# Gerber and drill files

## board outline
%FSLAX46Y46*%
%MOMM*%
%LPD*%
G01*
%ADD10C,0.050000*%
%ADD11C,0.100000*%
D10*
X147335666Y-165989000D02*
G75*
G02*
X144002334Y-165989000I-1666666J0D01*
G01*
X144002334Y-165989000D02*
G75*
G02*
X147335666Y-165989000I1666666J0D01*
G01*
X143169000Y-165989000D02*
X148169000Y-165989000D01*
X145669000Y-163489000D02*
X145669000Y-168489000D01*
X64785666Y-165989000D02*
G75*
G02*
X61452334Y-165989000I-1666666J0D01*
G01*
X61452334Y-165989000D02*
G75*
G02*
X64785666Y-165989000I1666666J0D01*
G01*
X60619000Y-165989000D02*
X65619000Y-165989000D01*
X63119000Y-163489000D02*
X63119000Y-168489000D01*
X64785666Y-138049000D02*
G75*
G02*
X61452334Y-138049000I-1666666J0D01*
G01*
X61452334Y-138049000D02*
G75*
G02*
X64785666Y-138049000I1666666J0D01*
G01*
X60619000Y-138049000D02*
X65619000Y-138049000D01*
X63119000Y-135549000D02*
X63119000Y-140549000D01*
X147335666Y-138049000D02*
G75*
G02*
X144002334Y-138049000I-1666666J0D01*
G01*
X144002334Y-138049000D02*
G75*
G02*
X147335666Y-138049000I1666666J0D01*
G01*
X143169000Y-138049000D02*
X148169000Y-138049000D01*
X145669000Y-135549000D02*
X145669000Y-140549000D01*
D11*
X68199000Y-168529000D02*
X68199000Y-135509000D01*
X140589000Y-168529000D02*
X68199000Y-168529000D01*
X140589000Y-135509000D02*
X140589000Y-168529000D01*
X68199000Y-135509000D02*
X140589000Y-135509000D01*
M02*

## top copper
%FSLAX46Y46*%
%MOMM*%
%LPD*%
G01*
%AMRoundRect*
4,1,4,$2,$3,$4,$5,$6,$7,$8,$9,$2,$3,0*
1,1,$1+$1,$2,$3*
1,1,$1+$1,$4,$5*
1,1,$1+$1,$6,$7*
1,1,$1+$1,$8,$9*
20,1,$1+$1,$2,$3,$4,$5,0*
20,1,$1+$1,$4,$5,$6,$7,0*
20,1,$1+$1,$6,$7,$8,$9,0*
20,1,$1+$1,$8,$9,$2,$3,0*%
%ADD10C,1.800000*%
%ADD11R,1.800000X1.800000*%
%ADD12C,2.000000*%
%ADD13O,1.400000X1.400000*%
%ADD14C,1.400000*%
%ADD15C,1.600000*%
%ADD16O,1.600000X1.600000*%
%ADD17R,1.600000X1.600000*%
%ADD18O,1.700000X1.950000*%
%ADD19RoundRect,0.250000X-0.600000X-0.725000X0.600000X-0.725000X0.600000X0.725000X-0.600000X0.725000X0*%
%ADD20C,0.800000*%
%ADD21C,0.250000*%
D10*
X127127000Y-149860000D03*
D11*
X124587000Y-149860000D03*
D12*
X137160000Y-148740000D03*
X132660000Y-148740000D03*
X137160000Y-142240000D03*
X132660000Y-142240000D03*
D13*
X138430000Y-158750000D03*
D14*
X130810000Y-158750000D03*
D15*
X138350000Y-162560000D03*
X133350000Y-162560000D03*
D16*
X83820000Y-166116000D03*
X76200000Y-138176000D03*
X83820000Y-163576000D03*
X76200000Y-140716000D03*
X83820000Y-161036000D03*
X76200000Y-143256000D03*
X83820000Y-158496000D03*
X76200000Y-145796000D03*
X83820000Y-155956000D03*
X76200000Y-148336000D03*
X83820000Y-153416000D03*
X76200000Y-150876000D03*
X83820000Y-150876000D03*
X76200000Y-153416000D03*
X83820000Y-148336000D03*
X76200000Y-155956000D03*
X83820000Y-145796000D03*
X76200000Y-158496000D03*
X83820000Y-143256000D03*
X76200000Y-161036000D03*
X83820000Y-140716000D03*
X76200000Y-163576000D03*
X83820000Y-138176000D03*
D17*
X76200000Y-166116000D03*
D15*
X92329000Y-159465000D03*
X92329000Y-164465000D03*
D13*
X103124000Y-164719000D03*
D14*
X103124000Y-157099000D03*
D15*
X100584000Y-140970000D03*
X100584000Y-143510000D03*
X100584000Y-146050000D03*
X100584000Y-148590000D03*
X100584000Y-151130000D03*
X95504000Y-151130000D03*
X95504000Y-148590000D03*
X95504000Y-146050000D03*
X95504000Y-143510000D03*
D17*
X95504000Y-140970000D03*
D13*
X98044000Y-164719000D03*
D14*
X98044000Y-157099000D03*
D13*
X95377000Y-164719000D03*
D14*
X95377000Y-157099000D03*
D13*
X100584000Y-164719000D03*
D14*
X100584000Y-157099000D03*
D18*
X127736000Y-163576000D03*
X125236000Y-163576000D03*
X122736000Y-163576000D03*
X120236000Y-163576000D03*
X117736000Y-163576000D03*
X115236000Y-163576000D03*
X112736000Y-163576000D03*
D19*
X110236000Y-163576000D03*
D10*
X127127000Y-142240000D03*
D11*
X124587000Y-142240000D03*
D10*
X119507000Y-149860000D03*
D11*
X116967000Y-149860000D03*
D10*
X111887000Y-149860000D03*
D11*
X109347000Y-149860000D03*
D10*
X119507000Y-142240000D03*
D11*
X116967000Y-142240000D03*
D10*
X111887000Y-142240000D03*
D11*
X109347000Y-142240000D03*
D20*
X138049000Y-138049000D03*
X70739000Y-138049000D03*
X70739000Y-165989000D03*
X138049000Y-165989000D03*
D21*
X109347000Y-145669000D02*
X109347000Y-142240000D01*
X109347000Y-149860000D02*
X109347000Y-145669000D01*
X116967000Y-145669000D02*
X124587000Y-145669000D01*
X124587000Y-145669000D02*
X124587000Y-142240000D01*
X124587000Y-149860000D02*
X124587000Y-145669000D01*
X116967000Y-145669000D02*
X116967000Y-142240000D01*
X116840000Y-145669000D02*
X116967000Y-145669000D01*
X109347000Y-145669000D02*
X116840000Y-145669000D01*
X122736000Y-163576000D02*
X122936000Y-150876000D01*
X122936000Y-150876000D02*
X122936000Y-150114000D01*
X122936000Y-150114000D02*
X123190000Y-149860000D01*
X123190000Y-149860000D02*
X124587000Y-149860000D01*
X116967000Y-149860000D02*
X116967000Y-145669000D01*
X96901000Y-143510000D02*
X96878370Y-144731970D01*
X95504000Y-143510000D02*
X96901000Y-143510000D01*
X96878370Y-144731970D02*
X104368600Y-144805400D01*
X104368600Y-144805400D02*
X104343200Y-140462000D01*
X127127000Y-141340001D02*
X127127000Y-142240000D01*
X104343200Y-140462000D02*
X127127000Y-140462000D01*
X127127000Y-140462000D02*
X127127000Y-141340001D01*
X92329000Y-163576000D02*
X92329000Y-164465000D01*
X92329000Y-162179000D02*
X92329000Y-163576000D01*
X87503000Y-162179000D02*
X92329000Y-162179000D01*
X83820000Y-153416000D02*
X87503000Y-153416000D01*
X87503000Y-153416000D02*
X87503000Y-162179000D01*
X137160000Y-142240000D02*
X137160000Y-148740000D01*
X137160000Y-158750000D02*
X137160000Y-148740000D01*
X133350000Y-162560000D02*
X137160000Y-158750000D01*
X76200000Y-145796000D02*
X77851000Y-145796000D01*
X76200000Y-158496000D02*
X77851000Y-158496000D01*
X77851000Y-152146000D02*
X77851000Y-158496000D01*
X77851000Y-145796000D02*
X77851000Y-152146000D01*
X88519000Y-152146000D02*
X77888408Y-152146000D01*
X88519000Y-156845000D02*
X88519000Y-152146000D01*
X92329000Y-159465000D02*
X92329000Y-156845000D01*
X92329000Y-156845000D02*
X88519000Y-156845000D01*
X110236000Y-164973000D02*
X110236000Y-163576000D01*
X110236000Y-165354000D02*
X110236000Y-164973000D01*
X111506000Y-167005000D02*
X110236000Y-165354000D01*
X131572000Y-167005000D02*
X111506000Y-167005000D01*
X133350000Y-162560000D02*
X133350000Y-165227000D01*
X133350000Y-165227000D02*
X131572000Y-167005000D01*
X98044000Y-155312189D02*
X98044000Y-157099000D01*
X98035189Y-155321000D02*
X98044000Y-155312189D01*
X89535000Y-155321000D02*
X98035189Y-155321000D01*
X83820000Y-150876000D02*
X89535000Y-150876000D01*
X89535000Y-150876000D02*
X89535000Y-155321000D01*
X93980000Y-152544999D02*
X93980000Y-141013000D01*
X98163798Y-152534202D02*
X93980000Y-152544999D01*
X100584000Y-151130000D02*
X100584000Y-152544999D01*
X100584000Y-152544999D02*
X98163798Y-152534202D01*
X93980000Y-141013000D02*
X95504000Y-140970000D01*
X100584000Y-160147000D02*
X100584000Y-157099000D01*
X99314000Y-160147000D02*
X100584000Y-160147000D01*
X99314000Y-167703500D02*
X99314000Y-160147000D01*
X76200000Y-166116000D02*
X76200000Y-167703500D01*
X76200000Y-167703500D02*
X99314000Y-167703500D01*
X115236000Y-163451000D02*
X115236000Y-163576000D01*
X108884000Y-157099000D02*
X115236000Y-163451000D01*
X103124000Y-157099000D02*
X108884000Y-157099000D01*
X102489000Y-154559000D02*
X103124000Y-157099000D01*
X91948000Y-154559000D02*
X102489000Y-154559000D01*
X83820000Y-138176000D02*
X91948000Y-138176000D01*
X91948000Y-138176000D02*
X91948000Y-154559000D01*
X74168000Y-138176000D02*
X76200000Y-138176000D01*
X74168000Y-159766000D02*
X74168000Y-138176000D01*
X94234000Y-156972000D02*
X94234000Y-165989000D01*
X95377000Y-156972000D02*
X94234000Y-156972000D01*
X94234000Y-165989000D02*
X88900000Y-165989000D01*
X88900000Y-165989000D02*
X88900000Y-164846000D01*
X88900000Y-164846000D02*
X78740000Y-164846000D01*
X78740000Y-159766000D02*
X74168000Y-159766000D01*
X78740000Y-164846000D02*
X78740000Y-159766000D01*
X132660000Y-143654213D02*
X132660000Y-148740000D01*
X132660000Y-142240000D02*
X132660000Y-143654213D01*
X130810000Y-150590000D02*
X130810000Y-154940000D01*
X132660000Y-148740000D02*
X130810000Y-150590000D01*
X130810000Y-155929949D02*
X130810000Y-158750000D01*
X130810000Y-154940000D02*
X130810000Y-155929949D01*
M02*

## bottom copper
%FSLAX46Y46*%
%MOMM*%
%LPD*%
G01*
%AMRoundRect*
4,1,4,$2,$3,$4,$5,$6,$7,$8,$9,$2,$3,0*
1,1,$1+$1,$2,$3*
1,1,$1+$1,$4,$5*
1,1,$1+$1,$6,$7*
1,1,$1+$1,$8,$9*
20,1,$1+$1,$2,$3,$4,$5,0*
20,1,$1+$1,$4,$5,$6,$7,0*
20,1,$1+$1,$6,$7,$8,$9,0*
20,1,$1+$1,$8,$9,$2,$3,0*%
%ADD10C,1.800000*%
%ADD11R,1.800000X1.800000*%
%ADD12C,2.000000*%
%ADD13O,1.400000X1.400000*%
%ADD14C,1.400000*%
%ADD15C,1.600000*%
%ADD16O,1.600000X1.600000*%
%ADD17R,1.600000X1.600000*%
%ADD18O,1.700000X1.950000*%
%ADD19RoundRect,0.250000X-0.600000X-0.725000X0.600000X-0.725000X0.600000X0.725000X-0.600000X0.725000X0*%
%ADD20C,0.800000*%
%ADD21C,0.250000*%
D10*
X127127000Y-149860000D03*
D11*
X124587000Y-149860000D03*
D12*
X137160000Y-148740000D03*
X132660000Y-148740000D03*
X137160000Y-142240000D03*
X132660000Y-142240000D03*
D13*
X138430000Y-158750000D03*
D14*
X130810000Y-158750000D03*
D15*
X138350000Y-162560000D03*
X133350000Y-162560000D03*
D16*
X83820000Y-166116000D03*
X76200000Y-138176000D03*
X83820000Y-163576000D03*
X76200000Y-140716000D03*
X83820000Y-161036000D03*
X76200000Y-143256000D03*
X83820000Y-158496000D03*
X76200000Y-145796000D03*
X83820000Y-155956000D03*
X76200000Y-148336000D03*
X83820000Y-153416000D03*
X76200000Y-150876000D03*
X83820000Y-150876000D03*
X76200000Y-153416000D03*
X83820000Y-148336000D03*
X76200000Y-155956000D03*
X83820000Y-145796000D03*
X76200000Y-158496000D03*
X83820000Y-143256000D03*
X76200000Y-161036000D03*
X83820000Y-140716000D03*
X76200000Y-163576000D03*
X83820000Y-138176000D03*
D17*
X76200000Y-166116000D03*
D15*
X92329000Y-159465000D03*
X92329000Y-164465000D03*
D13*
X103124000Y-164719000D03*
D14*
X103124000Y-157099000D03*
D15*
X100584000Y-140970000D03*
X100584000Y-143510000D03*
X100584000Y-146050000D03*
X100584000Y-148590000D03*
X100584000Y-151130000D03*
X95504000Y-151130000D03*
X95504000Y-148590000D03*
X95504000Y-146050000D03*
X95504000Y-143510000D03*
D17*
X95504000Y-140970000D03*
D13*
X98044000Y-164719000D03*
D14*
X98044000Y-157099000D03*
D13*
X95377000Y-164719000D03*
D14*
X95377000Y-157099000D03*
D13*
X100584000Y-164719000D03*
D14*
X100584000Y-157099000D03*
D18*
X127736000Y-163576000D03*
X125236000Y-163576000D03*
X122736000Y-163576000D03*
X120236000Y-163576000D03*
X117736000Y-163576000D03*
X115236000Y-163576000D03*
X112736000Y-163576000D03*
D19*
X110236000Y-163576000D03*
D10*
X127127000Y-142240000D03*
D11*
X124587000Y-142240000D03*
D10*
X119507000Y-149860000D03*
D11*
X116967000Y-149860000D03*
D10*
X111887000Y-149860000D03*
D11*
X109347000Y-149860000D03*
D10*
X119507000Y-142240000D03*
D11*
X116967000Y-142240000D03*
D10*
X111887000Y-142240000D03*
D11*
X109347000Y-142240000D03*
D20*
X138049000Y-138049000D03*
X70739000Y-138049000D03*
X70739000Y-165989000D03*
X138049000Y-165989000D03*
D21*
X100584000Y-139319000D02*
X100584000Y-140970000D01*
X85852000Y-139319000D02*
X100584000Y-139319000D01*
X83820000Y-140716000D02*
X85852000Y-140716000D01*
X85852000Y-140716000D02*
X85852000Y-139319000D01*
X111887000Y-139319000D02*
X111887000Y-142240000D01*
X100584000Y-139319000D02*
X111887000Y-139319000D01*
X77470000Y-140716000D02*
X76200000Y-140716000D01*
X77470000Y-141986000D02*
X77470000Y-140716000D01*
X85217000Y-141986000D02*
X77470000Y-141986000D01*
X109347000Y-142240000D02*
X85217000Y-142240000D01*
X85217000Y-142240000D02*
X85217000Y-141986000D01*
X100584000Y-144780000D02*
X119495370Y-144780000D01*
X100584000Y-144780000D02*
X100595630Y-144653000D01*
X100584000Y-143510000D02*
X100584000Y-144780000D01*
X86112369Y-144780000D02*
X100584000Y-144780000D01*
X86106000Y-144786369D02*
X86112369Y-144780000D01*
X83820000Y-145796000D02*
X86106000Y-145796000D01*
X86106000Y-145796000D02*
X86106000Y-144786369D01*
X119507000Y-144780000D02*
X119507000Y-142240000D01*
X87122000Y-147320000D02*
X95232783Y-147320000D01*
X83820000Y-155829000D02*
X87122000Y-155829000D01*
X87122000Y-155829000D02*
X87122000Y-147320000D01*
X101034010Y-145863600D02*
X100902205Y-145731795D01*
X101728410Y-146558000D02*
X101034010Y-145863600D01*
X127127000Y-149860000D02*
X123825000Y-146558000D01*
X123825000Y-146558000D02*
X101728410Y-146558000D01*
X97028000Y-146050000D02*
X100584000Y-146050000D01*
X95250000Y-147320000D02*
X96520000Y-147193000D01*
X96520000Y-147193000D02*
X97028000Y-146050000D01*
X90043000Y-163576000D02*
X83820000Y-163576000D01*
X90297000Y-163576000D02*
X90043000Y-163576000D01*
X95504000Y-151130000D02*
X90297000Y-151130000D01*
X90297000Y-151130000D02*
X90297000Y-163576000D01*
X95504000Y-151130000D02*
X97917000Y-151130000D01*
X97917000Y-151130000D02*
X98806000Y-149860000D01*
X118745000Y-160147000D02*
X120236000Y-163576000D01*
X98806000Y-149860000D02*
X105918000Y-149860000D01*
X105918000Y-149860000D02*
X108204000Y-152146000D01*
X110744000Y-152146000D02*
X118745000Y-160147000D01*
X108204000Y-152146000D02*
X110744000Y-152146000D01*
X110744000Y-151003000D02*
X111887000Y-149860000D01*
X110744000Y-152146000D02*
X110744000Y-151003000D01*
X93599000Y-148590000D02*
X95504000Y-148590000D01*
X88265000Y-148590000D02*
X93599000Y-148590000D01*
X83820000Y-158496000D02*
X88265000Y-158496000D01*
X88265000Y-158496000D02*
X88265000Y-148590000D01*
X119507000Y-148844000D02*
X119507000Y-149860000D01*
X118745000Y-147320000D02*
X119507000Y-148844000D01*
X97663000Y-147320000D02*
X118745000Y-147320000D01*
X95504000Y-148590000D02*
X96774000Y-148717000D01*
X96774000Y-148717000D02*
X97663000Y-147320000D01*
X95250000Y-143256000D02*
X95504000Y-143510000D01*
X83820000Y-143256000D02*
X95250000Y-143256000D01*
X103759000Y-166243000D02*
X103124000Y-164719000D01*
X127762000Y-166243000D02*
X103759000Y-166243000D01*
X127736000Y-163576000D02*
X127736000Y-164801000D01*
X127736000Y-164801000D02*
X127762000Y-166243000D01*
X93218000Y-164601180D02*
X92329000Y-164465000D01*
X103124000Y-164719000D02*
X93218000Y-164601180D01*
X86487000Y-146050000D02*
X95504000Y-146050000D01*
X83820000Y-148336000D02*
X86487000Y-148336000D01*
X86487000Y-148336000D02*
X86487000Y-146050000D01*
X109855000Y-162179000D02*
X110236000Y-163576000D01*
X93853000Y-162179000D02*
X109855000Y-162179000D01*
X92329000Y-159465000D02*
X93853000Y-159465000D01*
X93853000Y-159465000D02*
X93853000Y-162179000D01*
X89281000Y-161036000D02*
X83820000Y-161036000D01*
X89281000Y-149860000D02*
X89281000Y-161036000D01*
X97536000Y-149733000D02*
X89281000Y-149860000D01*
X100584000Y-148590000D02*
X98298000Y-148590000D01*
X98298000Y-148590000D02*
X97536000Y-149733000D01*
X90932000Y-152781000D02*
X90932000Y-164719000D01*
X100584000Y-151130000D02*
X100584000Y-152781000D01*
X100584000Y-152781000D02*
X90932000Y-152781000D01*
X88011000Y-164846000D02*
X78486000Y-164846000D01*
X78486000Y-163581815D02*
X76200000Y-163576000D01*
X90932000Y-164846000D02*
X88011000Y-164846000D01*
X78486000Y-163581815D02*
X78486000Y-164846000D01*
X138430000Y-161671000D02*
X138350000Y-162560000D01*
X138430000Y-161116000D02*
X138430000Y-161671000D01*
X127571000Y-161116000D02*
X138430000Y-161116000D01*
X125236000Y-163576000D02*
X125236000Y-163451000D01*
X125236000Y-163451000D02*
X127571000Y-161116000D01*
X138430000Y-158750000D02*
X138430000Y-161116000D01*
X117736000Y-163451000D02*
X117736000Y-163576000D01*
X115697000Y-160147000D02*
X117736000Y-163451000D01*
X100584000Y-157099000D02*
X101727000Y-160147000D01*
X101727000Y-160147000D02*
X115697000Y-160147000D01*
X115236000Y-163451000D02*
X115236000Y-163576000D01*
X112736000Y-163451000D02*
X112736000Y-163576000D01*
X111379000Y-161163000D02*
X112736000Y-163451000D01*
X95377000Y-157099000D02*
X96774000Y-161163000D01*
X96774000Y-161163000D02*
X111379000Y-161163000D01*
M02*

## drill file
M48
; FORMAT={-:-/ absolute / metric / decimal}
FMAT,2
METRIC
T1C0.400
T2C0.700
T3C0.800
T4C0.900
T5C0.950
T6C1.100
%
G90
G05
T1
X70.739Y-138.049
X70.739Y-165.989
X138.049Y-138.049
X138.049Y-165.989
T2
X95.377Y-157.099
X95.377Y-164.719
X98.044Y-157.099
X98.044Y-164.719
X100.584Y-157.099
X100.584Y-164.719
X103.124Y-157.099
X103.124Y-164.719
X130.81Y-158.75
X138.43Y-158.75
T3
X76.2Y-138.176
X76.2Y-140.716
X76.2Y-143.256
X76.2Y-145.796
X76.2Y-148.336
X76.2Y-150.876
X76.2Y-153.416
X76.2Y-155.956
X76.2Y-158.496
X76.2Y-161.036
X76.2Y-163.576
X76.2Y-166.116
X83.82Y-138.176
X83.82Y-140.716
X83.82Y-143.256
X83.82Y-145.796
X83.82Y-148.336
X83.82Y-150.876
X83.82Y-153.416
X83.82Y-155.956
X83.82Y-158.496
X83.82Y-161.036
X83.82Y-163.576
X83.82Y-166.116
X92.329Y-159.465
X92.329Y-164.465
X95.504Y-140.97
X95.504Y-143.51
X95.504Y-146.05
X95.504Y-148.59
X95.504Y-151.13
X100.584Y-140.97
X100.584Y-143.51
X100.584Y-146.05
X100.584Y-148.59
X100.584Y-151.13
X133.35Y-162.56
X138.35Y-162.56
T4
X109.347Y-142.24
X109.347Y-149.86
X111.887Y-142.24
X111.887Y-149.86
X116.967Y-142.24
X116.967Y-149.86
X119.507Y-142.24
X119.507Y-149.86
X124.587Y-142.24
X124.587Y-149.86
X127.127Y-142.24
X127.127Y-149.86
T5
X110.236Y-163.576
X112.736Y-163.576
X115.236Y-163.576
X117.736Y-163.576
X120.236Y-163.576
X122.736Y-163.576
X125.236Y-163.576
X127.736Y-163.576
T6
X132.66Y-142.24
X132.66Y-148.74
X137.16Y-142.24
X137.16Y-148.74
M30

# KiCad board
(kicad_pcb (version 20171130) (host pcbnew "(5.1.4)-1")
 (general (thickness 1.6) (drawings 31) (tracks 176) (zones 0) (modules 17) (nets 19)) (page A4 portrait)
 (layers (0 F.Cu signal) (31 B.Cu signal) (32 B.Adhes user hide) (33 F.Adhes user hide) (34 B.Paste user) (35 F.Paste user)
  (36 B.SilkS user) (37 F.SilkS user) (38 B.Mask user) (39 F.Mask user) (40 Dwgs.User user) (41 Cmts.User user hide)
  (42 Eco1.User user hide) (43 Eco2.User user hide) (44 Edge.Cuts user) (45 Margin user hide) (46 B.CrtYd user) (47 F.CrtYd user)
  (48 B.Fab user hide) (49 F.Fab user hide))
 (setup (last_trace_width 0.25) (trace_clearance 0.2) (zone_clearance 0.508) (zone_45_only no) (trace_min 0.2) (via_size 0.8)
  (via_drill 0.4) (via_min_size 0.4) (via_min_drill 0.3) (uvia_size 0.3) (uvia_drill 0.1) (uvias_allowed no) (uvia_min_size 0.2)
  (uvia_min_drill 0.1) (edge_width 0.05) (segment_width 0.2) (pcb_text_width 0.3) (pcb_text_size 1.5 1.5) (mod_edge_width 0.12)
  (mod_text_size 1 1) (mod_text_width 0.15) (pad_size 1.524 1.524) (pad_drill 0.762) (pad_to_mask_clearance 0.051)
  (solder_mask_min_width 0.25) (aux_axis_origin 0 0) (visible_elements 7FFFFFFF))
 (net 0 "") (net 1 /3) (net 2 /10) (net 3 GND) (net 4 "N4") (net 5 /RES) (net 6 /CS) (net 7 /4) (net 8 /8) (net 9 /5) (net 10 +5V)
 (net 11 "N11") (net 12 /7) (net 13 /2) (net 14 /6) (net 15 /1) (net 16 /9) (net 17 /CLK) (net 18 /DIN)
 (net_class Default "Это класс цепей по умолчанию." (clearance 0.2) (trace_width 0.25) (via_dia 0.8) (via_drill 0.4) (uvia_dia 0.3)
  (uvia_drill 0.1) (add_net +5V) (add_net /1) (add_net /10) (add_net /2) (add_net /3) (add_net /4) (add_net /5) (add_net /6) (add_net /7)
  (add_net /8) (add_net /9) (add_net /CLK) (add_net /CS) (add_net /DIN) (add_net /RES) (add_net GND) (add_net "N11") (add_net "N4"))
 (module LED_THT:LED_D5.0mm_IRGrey (layer F.Cu) (at 124.587 149.86)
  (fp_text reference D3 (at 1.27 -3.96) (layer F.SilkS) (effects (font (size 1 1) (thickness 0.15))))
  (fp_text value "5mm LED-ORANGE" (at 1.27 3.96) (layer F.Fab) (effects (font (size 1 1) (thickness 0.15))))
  (pad 2 thru_hole circle (at 2.54 0) (size 1.8 1.8) (drill 0.9) (layers *.Cu *.Mask) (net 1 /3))
  (pad 1 thru_hole rect (at 0 0) (size 1.8 1.8) (drill 0.9) (layers *.Cu *.Mask) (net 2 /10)))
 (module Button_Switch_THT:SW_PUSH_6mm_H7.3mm (layer F.Cu) (at 137.16 142.24 270)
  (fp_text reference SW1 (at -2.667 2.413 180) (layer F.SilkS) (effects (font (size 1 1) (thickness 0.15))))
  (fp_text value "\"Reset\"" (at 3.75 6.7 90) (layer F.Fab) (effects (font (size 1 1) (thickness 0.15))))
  (pad 1 thru_hole circle (at 6.5 0) (size 2 2) (drill 1.1) (layers *.Cu *.Mask) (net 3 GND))
  (pad 2 thru_hole circle (at 6.5 4.5) (size 2 2) (drill 1.1) (layers *.Cu *.Mask) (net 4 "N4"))
  (pad 1 thru_hole circle (at 0 0) (size 2 2) (drill 1.1) (layers *.Cu *.Mask) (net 3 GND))
  (pad 2 thru_hole circle (at 0 4.5) (size 2 2) (drill 1.1) (layers *.Cu *.Mask) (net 4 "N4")))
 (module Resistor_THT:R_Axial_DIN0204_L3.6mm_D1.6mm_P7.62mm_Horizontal (layer B.Cu) (at 130.81 158.75)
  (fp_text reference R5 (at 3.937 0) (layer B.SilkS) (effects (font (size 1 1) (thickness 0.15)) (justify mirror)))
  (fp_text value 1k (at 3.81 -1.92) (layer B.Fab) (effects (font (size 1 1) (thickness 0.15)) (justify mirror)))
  (pad 2 thru_hole oval (at 7.62 0) (size 1.4 1.4) (drill 0.7) (layers *.Cu *.Mask) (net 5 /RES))
  (pad 1 thru_hole circle (at 0 0) (size 1.4 1.4) (drill 0.7) (layers *.Cu *.Mask) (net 4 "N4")))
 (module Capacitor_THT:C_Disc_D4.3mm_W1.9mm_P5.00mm (layer B.Cu) (at 133.35 162.56)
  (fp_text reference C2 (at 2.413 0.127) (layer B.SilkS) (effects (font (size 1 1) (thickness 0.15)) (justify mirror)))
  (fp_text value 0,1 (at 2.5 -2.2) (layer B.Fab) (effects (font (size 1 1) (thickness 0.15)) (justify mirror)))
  (pad 2 thru_hole circle (at 5 0) (size 1.6 1.6) (drill 0.8) (layers *.Cu *.Mask) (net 5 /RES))
  (pad 1 thru_hole circle (at 0 0) (size 1.6 1.6) (drill 0.8) (layers *.Cu *.Mask) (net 3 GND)))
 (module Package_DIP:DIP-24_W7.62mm (layer B.Cu) (at 76.2 166.116)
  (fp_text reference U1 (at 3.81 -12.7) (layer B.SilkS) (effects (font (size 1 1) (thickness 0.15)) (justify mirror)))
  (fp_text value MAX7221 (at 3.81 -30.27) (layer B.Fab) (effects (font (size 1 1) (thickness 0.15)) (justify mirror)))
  (pad 24 thru_hole oval (at 7.62 0) (size 1.6 1.6) (drill 0.8) (layers *.Cu *.Mask))
  (pad 12 thru_hole oval (at 0 -27.94) (size 1.6 1.6) (drill 0.8) (layers *.Cu *.Mask) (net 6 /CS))
  (pad 23 thru_hole oval (at 7.62 -2.54) (size 1.6 1.6) (drill 0.8) (layers *.Cu *.Mask) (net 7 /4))
  (pad 11 thru_hole oval (at 0 -25.4) (size 1.6 1.6) (drill 0.8) (layers *.Cu *.Mask) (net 2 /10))
  (pad 22 thru_hole oval (at 7.62 -5.08) (size 1.6 1.6) (drill 0.8) (layers *.Cu *.Mask) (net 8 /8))
  (pad 10 thru_hole oval (at 0 -22.86) (size 1.6 1.6) (drill 0.8) (layers *.Cu *.Mask))
  (pad 21 thru_hole oval (at 7.62 -7.62) (size 1.6 1.6) (drill 0.8) (layers *.Cu *.Mask) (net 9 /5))
  (pad 9 thru_hole oval (at 0 -20.32) (size 1.6 1.6) (drill 0.8) (layers *.Cu *.Mask) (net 3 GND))
  (pad 20 thru_hole oval (at 7.62 -10.16) (size 1.6 1.6) (drill 0.8) (layers *.Cu *.Mask) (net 1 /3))
  (pad 8 thru_hole oval (at 0 -17.78) (size 1.6 1.6) (drill 0.8) (layers *.Cu *.Mask))
  (pad 19 thru_hole oval (at 7.62 -12.7) (size 1.6 1.6) (drill 0.8) (layers *.Cu *.Mask) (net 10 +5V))
  (pad 7 thru_hole oval (at 0 -15.24) (size 1.6 1.6) (drill 0.8) (layers *.Cu *.Mask))
  (pad 18 thru_hole oval (at 7.62 -15.24) (size 1.6 1.6) (drill 0.8) (layers *.Cu *.Mask) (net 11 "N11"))
  (pad 6 thru_hole oval (at 0 -12.7) (size 1.6 1.6) (drill 0.8) (layers *.Cu *.Mask))
  (pad 17 thru_hole oval (at 7.62 -17.78) (size 1.6 1.6) (drill 0.8) (layers *.Cu *.Mask) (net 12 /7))
  (pad 5 thru_hole oval (at 0 -10.16) (size 1.6 1.6) (drill 0.8) (layers *.Cu *.Mask))
  (pad 16 thru_hole oval (at 7.62 -20.32) (size 1.6 1.6) (drill 0.8) (layers *.Cu *.Mask) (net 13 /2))
  (pad 4 thru_hole oval (at 0 -7.62) (size 1.6 1.6) (drill 0.8) (layers *.Cu *.Mask) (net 3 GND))
  (pad 15 thru_hole oval (at 7.62 -22.86) (size 1.6 1.6) (drill 0.8) (layers *.Cu *.Mask) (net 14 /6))
  (pad 3 thru_hole oval (at 0 -5.08) (size 1.6 1.6) (drill 0.8) (layers *.Cu *.Mask))
  (pad 14 thru_hole oval (at 7.62 -25.4) (size 1.6 1.6) (drill 0.8) (layers *.Cu *.Mask) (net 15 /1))
  (pad 2 thru_hole oval (at 0 -2.54) (size 1.6 1.6) (drill 0.8) (layers *.Cu *.Mask) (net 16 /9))
  (pad 13 thru_hole oval (at 7.62 -27.94) (size 1.6 1.6) (drill 0.8) (layers *.Cu *.Mask) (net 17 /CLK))
  (pad 1 thru_hole rect (at 0 0) (size 1.6 1.6) (drill 0.8) (layers *.Cu *.Mask) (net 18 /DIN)))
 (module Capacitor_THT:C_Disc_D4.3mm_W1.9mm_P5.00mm (layer B.Cu) (at 92.329 164.465 90)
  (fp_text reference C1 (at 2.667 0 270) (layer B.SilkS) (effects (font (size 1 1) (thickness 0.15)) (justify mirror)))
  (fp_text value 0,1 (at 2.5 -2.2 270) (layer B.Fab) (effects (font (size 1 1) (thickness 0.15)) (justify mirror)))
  (pad 2 thru_hole circle (at 5 0 90) (size 1.6 1.6) (drill 0.8) (layers *.Cu *.Mask) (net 3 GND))
  (pad 1 thru_hole circle (at 0 0 90) (size 1.6 1.6) (drill 0.8) (layers *.Cu *.Mask) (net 10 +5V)))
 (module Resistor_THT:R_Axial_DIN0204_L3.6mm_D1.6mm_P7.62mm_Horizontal (layer B.Cu) (at 103.124 157.099 270)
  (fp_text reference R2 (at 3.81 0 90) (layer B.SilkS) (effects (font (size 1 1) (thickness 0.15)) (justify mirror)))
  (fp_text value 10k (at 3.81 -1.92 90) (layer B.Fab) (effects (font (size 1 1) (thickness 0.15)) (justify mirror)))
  (pad 2 thru_hole oval (at 7.62 0 270) (size 1.4 1.4) (drill 0.7) (layers *.Cu *.Mask) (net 10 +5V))
  (pad 1 thru_hole circle (at 0 0 270) (size 1.4 1.4) (drill 0.7) (layers *.Cu *.Mask) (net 17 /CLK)))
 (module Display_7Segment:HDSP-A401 (layer F.Cu) (at 95.504 140.97)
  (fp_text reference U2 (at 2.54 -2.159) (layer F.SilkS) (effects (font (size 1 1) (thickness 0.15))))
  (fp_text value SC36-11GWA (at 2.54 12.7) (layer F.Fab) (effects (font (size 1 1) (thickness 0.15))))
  (pad 10 thru_hole circle (at 5.08 0) (size 1.6 1.6) (drill 0.8) (layers *.Cu *.Mask) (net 15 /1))
  (pad 9 thru_hole circle (at 5.08 2.54) (size 1.6 1.6) (drill 0.8) (layers *.Cu *.Mask) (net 13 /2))
  (pad 8 thru_hole circle (at 5.08 5.08) (size 1.6 1.6) (drill 0.8) (layers *.Cu *.Mask) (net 1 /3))
  (pad 7 thru_hole circle (at 5.08 7.62) (size 1.6 1.6) (drill 0.8) (layers *.Cu *.Mask) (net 8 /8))
  (pad 6 thru_hole circle (at 5.08 10.16) (size 1.6 1.6) (drill 0.8) (layers *.Cu *.Mask) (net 16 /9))
  (pad 5 thru_hole circle (at 0 10.16) (size 1.6 1.6) (drill 0.8) (layers *.Cu *.Mask) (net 7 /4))
  (pad 4 thru_hole circle (at 0 7.62) (size 1.6 1.6) (drill 0.8) (layers *.Cu *.Mask) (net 9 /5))
  (pad 3 thru_hole circle (at 0 5.08) (size 1.6 1.6) (drill 0.8) (layers *.Cu *.Mask) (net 12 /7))
  (pad 2 thru_hole circle (at 0 2.54) (size 1.6 1.6) (drill 0.8) (layers *.Cu *.Mask) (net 14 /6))
  (pad 1 thru_hole rect (at 0 0) (size 1.6 1.6) (drill 0.8) (layers *.Cu *.Mask) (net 16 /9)))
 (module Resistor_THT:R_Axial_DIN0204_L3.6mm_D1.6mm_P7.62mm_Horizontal (layer B.Cu) (at 98.044 157.099 270)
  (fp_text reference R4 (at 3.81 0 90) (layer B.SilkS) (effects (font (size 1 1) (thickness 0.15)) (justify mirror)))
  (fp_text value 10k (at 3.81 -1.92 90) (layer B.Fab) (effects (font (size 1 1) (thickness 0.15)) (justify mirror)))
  (pad 2 thru_hole oval (at 7.62 0 270) (size 1.4 1.4) (drill 0.7) (layers *.Cu *.Mask) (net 10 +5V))
  (pad 1 thru_hole circle (at 0 0 270) (size 1.4 1.4) (drill 0.7) (layers *.Cu *.Mask) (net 11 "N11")))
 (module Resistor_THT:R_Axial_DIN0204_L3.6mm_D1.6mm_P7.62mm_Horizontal (layer B.Cu) (at 95.377 157.099 270)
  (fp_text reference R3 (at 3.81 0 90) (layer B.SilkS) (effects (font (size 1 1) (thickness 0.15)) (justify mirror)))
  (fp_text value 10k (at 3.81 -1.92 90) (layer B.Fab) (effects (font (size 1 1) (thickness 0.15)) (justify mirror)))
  (pad 2 thru_hole oval (at 7.62 0 270) (size 1.4 1.4) (drill 0.7) (layers *.Cu *.Mask) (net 10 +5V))
  (pad 1 thru_hole circle (at 0 0 270) (size 1.4 1.4) (drill 0.7) (layers *.Cu *.Mask) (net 6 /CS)))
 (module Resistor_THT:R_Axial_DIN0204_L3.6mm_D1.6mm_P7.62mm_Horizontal (layer B.Cu) (at 100.584 157.099 270)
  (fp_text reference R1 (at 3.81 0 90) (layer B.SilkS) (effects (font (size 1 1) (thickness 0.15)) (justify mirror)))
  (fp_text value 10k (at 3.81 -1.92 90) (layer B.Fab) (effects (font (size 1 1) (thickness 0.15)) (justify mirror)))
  (pad 2 thru_hole oval (at 7.62 0 270) (size 1.4 1.4) (drill 0.7) (layers *.Cu *.Mask) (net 10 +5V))
  (pad 1 thru_hole circle (at 0 0 270) (size 1.4 1.4) (drill 0.7) (layers *.Cu *.Mask) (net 18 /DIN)))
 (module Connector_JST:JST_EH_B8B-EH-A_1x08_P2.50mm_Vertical (layer B.Cu) (at 110.236 163.576)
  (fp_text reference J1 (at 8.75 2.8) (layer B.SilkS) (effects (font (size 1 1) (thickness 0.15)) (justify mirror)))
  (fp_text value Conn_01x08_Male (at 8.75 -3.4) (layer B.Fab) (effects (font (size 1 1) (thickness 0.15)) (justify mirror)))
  (pad 8 thru_hole oval (at 17.5 0) (size 1.7 1.95) (drill 0.95) (layers *.Cu *.Mask) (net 10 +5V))
  (pad 7 thru_hole oval (at 15 0) (size 1.7 1.95) (drill 0.95) (layers *.Cu *.Mask) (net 5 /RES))
  (pad 6 thru_hole oval (at 12.5 0) (size 1.7 1.95) (drill 0.95) (layers *.Cu *.Mask) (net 2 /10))
  (pad 5 thru_hole oval (at 10 0) (size 1.7 1.95) (drill 0.95) (layers *.Cu *.Mask) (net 7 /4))
  (pad 4 thru_hole oval (at 7.5 0) (size 1.7 1.95) (drill 0.95) (layers *.Cu *.Mask) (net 18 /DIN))
  (pad 3 thru_hole oval (at 5 0) (size 1.7 1.95) (drill 0.95) (layers *.Cu *.Mask) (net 17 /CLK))
  (pad 2 thru_hole oval (at 2.5 0) (size 1.7 1.95) (drill 0.95) (layers *.Cu *.Mask) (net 6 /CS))
  (pad 1 thru_hole roundrect (at 0 0) (size 1.7 1.95) (drill 0.95) (layers *.Cu *.Mask) (roundrect_rratio 0.147059) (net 3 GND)))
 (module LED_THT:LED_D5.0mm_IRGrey (layer F.Cu) (at 124.587 142.24)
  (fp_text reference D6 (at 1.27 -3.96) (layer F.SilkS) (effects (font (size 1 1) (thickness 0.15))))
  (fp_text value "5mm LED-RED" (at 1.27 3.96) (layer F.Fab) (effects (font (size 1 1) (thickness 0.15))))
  (pad 2 thru_hole circle (at 2.54 0) (size 1.8 1.8) (drill 0.9) (layers *.Cu *.Mask) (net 14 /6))
  (pad 1 thru_hole rect (at 0 0) (size 1.8 1.8) (drill 0.9) (layers *.Cu *.Mask) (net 2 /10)))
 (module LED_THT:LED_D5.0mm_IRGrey (layer F.Cu) (at 116.967 149.86)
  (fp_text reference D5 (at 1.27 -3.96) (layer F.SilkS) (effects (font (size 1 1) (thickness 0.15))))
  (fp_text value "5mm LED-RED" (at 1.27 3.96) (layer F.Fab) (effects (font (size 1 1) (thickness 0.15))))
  (pad 2 thru_hole circle (at 2.54 0) (size 1.8 1.8) (drill 0.9) (layers *.Cu *.Mask) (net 9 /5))
  (pad 1 thru_hole rect (at 0 0) (size 1.8 1.8) (drill 0.9) (layers *.Cu *.Mask) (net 2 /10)))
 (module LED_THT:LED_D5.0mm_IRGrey (layer F.Cu) (at 109.347 149.86)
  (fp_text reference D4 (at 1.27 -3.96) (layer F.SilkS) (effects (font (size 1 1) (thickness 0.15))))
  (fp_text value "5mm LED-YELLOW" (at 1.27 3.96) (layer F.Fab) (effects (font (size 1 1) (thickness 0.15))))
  (pad 2 thru_hole circle (at 2.54 0) (size 1.8 1.8) (drill 0.9) (layers *.Cu *.Mask) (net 7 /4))
  (pad 1 thru_hole rect (at 0 0) (size 1.8 1.8) (drill 0.9) (layers *.Cu *.Mask) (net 2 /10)))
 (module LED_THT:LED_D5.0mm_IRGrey (layer F.Cu) (at 116.967 142.24)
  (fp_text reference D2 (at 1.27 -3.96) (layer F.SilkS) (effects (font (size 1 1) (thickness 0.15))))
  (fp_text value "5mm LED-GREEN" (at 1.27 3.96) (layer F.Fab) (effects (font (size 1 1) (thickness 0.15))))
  (pad 2 thru_hole circle (at 2.54 0) (size 1.8 1.8) (drill 0.9) (layers *.Cu *.Mask) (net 13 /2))
  (pad 1 thru_hole rect (at 0 0) (size 1.8 1.8) (drill 0.9) (layers *.Cu *.Mask) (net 2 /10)))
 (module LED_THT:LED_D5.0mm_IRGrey (layer F.Cu) (at 109.347 142.24)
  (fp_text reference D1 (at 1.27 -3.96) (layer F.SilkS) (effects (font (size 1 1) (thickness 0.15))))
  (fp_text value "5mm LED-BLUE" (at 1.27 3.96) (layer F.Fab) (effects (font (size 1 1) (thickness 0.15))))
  (pad 2 thru_hole circle (at 2.54 0) (size 1.8 1.8) (drill 0.9) (layers *.Cu *.Mask) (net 15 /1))
  (pad 1 thru_hole rect (at 0 0) (size 1.8 1.8) (drill 0.9) (layers *.Cu *.Mask) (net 2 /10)))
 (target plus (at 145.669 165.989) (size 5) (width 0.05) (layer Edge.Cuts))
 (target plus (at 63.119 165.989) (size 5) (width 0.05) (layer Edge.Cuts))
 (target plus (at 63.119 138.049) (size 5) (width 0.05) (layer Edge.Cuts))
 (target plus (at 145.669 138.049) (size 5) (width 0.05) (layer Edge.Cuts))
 (gr_line (start 68.199 168.529) (end 68.199 135.509) (layer Edge.Cuts) (width 0.1))
 (gr_line (start 140.589 168.529) (end 68.199 168.529) (layer Edge.Cuts) (width 0.1))
 (gr_line (start 140.589 135.509) (end 140.589 168.529) (layer Edge.Cuts) (width 0.1))
 (gr_line (start 68.199 135.509) (end 140.589 135.509) (layer Edge.Cuts) (width 0.1))
 (via (at 138.049 138.049) (size 0.8) (drill 0.4) (layers F.Cu B.Cu) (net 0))
 (via (at 70.739 138.049) (size 0.8) (drill 0.4) (layers F.Cu B.Cu) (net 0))
 (via (at 70.739 165.989) (size 0.8) (drill 0.4) (layers F.Cu B.Cu) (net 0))
 (via (at 138.049 165.989) (size 0.8) (drill 0.4) (layers F.Cu B.Cu) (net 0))
 (segment (start 100.584 139.319) (end 100.584 140.97) (width 0.25) (layer B.Cu) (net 15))
 (segment (start 85.852 139.319) (end 100.584 139.319) (width 0.25) (layer B.Cu) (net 15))
 (segment (start 83.82 140.716) (end 85.852 140.716) (width 0.25) (layer B.Cu) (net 15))
 (segment (start 85.852 140.716) (end 85.852 139.319) (width 0.25) (layer B.Cu) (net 15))
 (segment (start 111.887 139.319) (end 111.887 142.24) (width 0.25) (layer B.Cu) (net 15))
 (segment (start 100.584 139.319) (end 111.887 139.319) (width 0.25) (layer B.Cu) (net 15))
 (segment (start 109.347 145.669) (end 109.347 142.24) (width 0.25) (layer F.Cu) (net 2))
 (segment (start 109.347 149.86) (end 109.347 145.669) (width 0.25) (layer F.Cu) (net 2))
 (segment (start 116.967 145.669) (end 124.587 145.669) (width 0.25) (layer F.Cu) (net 2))
 (segment (start 124.587 145.669) (end 124.587 142.24) (width 0.25) (layer F.Cu) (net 2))
 (segment (start 124.587 149.86) (end 124.587 145.669) (width 0.25) (layer F.Cu) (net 2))
 (segment (start 116.967 145.669) (end 116.967 142.24) (width 0.25) (layer F.Cu) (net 2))
 (segment (start 77.47 140.716) (end 76.2 140.716) (width 0.25) (layer B.Cu) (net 2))
 (segment (start 77.47 141.986) (end 77.47 140.716) (width 0.25) (layer B.Cu) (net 2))
 (segment (start 85.217 141.986) (end 77.47 141.986) (width 0.25) (layer B.Cu) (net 2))
 (segment (start 109.347 142.24) (end 85.217 142.24) (width 0.25) (layer B.Cu) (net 2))
 (segment (start 85.217 142.24) (end 85.217 141.986) (width 0.25) (layer B.Cu) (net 2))
 (segment (start 116.84 145.669) (end 116.967 145.669) (width 0.25) (layer F.Cu) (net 2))
 (segment (start 109.347 145.669) (end 116.84 145.669) (width 0.25) (layer F.Cu) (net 2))
 (segment (start 122.736 163.576) (end 122.936 150.876) (width 0.25) (layer F.Cu) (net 2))
 (segment (start 122.936 150.876) (end 122.936 150.114) (width 0.25) (layer F.Cu) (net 2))
 (segment (start 122.936 150.114) (end 123.19 149.86) (width 0.25) (layer F.Cu) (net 2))
 (segment (start 123.19 149.86) (end 124.587 149.86) (width 0.25) (layer F.Cu) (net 2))
 (segment (start 116.967 149.86) (end 116.967 145.669) (width 0.25) (layer F.Cu) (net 2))
 (segment (start 100.584 144.78) (end 119.49537 144.78) (width 0.25) (layer B.Cu) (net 13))
 (segment (start 100.584 144.78) (end 100.59563 144.653) (width 0.25) (layer B.Cu) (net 13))
 (segment (start 100.584 143.51) (end 100.584 144.78) (width 0.25) (layer B.Cu) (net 13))
 (segment (start 86.112369 144.78) (end 100.584 144.78) (width 0.25) (layer B.Cu) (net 13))
 (segment (start 86.106 144.786369) (end 86.112369 144.78) (width 0.25) (layer B.Cu) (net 13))
 (segment (start 83.82 145.796) (end 86.106 145.796) (width 0.25) (layer B.Cu) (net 13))
 (segment (start 86.106 145.796) (end 86.106 144.786369) (width 0.25) (layer B.Cu) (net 13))
 (segment (start 119.507 144.78) (end 119.507 142.24) (width 0.25) (layer B.Cu) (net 13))
 (segment (start 87.122 147.32) (end 95.232783 147.32) (width 0.25) (layer B.Cu) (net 1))
 (segment (start 83.82 155.829) (end 87.122 155.829) (width 0.25) (layer B.Cu) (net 1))
 (segment (start 87.122 155.829) (end 87.122 147.32) (width 0.25) (layer B.Cu) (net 1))
 (segment (start 101.03401 145.8636) (end 100.902205 145.731795) (width 0.25) (layer B.Cu) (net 1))
 (segment (start 101.72841 146.558) (end 101.03401 145.8636) (width 0.25) (layer B.Cu) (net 1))
 (segment (start 127.127 149.86) (end 123.825 146.558) (width 0.25) (layer B.Cu) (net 1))
 (segment (start 123.825 146.558) (end 101.72841 146.558) (width 0.25) (layer B.Cu) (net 1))
 (segment (start 97.028 146.05) (end 100.584 146.05) (width 0.25) (layer B.Cu) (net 1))
 (segment (start 95.25 147.32) (end 96.52 147.193) (width 0.25) (layer B.Cu) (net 1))
 (segment (start 96.52 147.193) (end 97.028 146.05) (width 0.25) (layer B.Cu) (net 1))
 (segment (start 90.043 163.576) (end 83.82 163.576) (width 0.25) (layer B.Cu) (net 7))
 (segment (start 90.297 163.576) (end 90.043 163.576) (width 0.25) (layer B.Cu) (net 7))
 (segment (start 95.504 151.13) (end 90.297 151.13) (width 0.25) (layer B.Cu) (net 7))
 (segment (start 90.297 151.13) (end 90.297 163.576) (width 0.25) (layer B.Cu) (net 7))
 (segment (start 95.504 151.13) (end 97.917 151.13) (width 0.25) (layer B.Cu) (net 7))
 (segment (start 97.917 151.13) (end 98.806 149.86) (width 0.25) (layer B.Cu) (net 7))
 (segment (start 118.745 160.147) (end 120.236 163.576) (width 0.25) (layer B.Cu) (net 7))
 (segment (start 98.806 149.86) (end 105.918 149.86) (width 0.25) (layer B.Cu) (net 7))
 (segment (start 105.918 149.86) (end 108.204 152.146) (width 0.25) (layer B.Cu) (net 7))
 (segment (start 110.744 152.146) (end 118.745 160.147) (width 0.25) (layer B.Cu) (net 7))
 (segment (start 108.204 152.146) (end 110.744 152.146) (width 0.25) (layer B.Cu) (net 7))
 (segment (start 110.744 151.003) (end 111.887 149.86) (width 0.25) (layer B.Cu) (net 7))
 (segment (start 110.744 152.146) (end 110.744 151.003) (width 0.25) (layer B.Cu) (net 7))
 (segment (start 93.599 148.59) (end 95.504 148.59) (width 0.25) (layer B.Cu) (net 9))
 (segment (start 88.265 148.59) (end 93.599 148.59) (width 0.25) (layer B.Cu) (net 9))
 (segment (start 83.82 158.496) (end 88.265 158.496) (width 0.25) (layer B.Cu) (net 9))
 (segment (start 88.265 158.496) (end 88.265 148.59) (width 0.25) (layer B.Cu) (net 9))
 (segment (start 119.507 148.844) (end 119.507 149.86) (width 0.25) (layer B.Cu) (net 9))
 (segment (start 118.745 147.32) (end 119.507 148.844) (width 0.25) (layer B.Cu) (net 9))
 (segment (start 97.663 147.32) (end 118.745 147.32) (width 0.25) (layer B.Cu) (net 9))
 (segment (start 95.504 148.59) (end 96.774 148.717) (width 0.25) (layer B.Cu) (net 9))
 (segment (start 96.774 148.717) (end 97.663 147.32) (width 0.25) (layer B.Cu) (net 9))
 (segment (start 95.25 143.256) (end 95.504 143.51) (width 0.25) (layer B.Cu) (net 14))
 (segment (start 83.82 143.256) (end 95.25 143.256) (width 0.25) (layer B.Cu) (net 14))
 (segment (start 96.901 143.51) (end 96.87837 144.73197) (width 0.25) (layer F.Cu) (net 14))
 (segment (start 95.504 143.51) (end 96.901 143.51) (width 0.25) (layer F.Cu) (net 14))
 (segment (start 96.87837 144.73197) (end 104.3686 144.8054) (width 0.25) (layer F.Cu) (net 14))
 (segment (start 104.3686 144.8054) (end 104.3432 140.462) (width 0.25) (layer F.Cu) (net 14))
 (segment (start 127.127 141.340001) (end 127.127 142.24) (width 0.25) (layer F.Cu) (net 14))
 (segment (start 104.3432 140.462) (end 127.127 140.462) (width 0.25) (layer F.Cu) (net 14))
 (segment (start 127.127 140.462) (end 127.127 141.340001) (width 0.25) (layer F.Cu) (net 14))
 (segment (start 92.329 163.576) (end 92.329 164.465) (width 0.25) (layer F.Cu) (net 10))
 (segment (start 92.329 162.179) (end 92.329 163.576) (width 0.25) (layer F.Cu) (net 10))
 (segment (start 87.503 162.179) (end 92.329 162.179) (width 0.25) (layer F.Cu) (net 10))
 (segment (start 83.82 153.416) (end 87.503 153.416) (width 0.25) (layer F.Cu) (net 10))
 (segment (start 87.503 153.416) (end 87.503 162.179) (width 0.25) (layer F.Cu) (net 10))
 (segment (start 103.759 166.243) (end 103.124 164.719) (width 0.25) (layer B.Cu) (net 10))
 (segment (start 127.762 166.243) (end 103.759 166.243) (width 0.25) (layer B.Cu) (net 10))
 (segment (start 127.736 163.576) (end 127.736 164.801) (width 0.25) (layer B.Cu) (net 10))
 (segment (start 127.736 164.801) (end 127.762 166.243) (width 0.25) (layer B.Cu) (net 10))
 (segment (start 93.218 164.60118) (end 92.329 164.465) (width 0.25) (layer B.Cu) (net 10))
 (segment (start 103.124 164.719) (end 93.218 164.60118) (width 0.25) (layer B.Cu) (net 10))
 (segment (start 86.487 146.05) (end 95.504 146.05) (width 0.25) (layer B.Cu) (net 12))
 (segment (start 83.82 148.336) (end 86.487 148.336) (width 0.25) (layer B.Cu) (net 12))
 (segment (start 86.487 148.336) (end 86.487 146.05) (width 0.25) (layer B.Cu) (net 12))
 (segment (start 137.16 142.24) (end 137.16 148.74) (width 0.25) (layer F.Cu) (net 3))
 (segment (start 137.16 158.75) (end 137.16 148.74) (width 0.25) (layer F.Cu) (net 3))
 (segment (start 133.35 162.56) (end 137.16 158.75) (width 0.25) (layer F.Cu) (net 3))
 (segment (start 76.2 145.796) (end 77.851 145.796) (width 0.25) (layer F.Cu) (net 3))
 (segment (start 76.2 158.496) (end 77.851 158.496) (width 0.25) (layer F.Cu) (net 3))
 (segment (start 77.851 152.146) (end 77.851 158.496) (width 0.25) (layer F.Cu) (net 3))
 (segment (start 77.851 145.796) (end 77.851 152.146) (width 0.25) (layer F.Cu) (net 3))
 (segment (start 88.519 152.146) (end 77.888408 152.146) (width 0.25) (layer F.Cu) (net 3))
 (segment (start 88.519 156.845) (end 88.519 152.146) (width 0.25) (layer F.Cu) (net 3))
 (segment (start 92.329 159.465) (end 92.329 156.845) (width 0.25) (layer F.Cu) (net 3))
 (segment (start 92.329 156.845) (end 88.519 156.845) (width 0.25) (layer F.Cu) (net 3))
 (segment (start 110.236 164.973) (end 110.236 163.576) (width 0.25) (layer F.Cu) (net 3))
 (segment (start 110.236 165.354) (end 110.236 164.973) (width 0.25) (layer F.Cu) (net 3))
 (segment (start 111.506 167.005) (end 110.236 165.354) (width 0.25) (layer F.Cu) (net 3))
 (segment (start 131.572 167.005) (end 111.506 167.005) (width 0.25) (layer F.Cu) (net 3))
 (segment (start 133.35 162.56) (end 133.35 165.227) (width 0.25) (layer F.Cu) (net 3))
 (segment (start 133.35 165.227) (end 131.572 167.005) (width 0.25) (layer F.Cu) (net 3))
 (segment (start 109.855 162.179) (end 110.236 163.576) (width 0.25) (layer B.Cu) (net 3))
 (segment (start 93.853 162.179) (end 109.855 162.179) (width 0.25) (layer B.Cu) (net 3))
 (segment (start 92.329 159.465) (end 93.853 159.465) (width 0.25) (layer B.Cu) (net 3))
 (segment (start 93.853 159.465) (end 93.853 162.179) (width 0.25) (layer B.Cu) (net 3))
 (segment (start 98.044 155.312189) (end 98.044 157.099) (width 0.25) (layer F.Cu) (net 11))
 (segment (start 98.035189 155.321) (end 98.044 155.312189) (width 0.25) (layer F.Cu) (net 11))
 (segment (start 89.535 155.321) (end 98.035189 155.321) (width 0.25) (layer F.Cu) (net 11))
 (segment (start 83.82 150.876) (end 89.535 150.876) (width 0.25) (layer F.Cu) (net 11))
 (segment (start 89.535 150.876) (end 89.535 155.321) (width 0.25) (layer F.Cu) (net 11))
 (segment (start 89.281 161.036) (end 83.82 161.036) (width 0.25) (layer B.Cu) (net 8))
 (segment (start 89.281 149.86) (end 89.281 161.036) (width 0.25) (layer B.Cu) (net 8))
 (segment (start 97.536 149.733) (end 89.281 149.86) (width 0.25) (layer B.Cu) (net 8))
 (segment (start 100.584 148.59) (end 98.298 148.59) (width 0.25) (layer B.Cu) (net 8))
 (segment (start 98.298 148.59) (end 97.536 149.733) (width 0.25) (layer B.Cu) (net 8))
 (segment (start 93.98 152.544999) (end 93.98 141.013) (width 0.25) (layer F.Cu) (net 16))
 (segment (start 98.163798 152.534202) (end 93.98 152.544999) (width 0.25) (layer F.Cu) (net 16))
 (segment (start 100.584 151.13) (end 100.584 152.544999) (width 0.25) (layer F.Cu) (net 16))
 (segment (start 100.584 152.544999) (end 98.163798 152.534202) (width 0.25) (layer F.Cu) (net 16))
 (segment (start 93.98 141.013) (end 95.504 140.97) (width 0.25) (layer F.Cu) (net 16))
 (segment (start 90.932 152.781) (end 90.932 164.719) (width 0.25) (layer B.Cu) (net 16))
 (segment (start 100.584 151.13) (end 100.584 152.781) (width 0.25) (layer B.Cu) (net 16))
 (segment (start 100.584 152.781) (end 90.932 152.781) (width 0.25) (layer B.Cu) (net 16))
 (segment (start 88.011 164.846) (end 78.486 164.846) (width 0.25) (layer B.Cu) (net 16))
 (segment (start 78.486 163.581815) (end 76.2 163.576) (width 0.25) (layer B.Cu) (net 16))
 (segment (start 90.932 164.846) (end 88.011 164.846) (width 0.25) (layer B.Cu) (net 16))
 (segment (start 78.486 163.581815) (end 78.486 164.846) (width 0.25) (layer B.Cu) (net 16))
 (segment (start 138.43 161.671) (end 138.35 162.56) (width 0.25) (layer B.Cu) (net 5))
 (segment (start 138.43 161.116) (end 138.43 161.671) (width 0.25) (layer B.Cu) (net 5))
 (segment (start 127.571 161.116) (end 138.43 161.116) (width 0.25) (layer B.Cu) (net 5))
 (segment (start 125.236 163.576) (end 125.236 163.451) (width 0.25) (layer B.Cu) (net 5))
 (segment (start 125.236 163.451) (end 127.571 161.116) (width 0.25) (layer B.Cu) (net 5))
 (segment (start 138.43 158.75) (end 138.43 161.116) (width 0.25) (layer B.Cu) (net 5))
 (segment (start 100.584 160.147) (end 100.584 157.099) (width 0.25) (layer F.Cu) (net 18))
 (segment (start 99.314 160.147) (end 100.584 160.147) (width 0.25) (layer F.Cu) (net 18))
 (segment (start 99.314 167.7035) (end 99.314 160.147) (width 0.25) (layer F.Cu) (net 18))
 (segment (start 76.2 166.116) (end 76.2 167.7035) (width 0.25) (layer F.Cu) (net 18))
 (segment (start 76.2 167.7035) (end 99.314 167.7035) (width 0.25) (layer F.Cu) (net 18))
 (segment (start 117.736 163.451) (end 117.736 163.576) (width 0.25) (layer B.Cu) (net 18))
 (segment (start 115.697 160.147) (end 117.736 163.451) (width 0.25) (layer B.Cu) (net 18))
 (segment (start 100.584 157.099) (end 101.727 160.147) (width 0.25) (layer B.Cu) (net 18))
 (segment (start 101.727 160.147) (end 115.697 160.147) (width 0.25) (layer B.Cu) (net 18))
 (segment (start 115.236 163.451) (end 115.236 163.576) (width 0.25) (layer B.Cu) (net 17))
 (segment (start 115.236 163.451) (end 115.236 163.576) (width 0.25) (layer F.Cu) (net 17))
 (segment (start 108.884 157.099) (end 115.236 163.451) (width 0.25) (layer F.Cu) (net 17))
 (segment (start 103.124 157.099) (end 108.884 157.099) (width 0.25) (layer F.Cu) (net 17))
 (segment (start 102.489 154.559) (end 103.124 157.099) (width 0.25) (layer F.Cu) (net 17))
 (segment (start 91.948 154.559) (end 102.489 154.559) (width 0.25) (layer F.Cu) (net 17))
 (segment (start 83.82 138.176) (end 91.948 138.176) (width 0.25) (layer F.Cu) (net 17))
 (segment (start 91.948 138.176) (end 91.948 154.559) (width 0.25) (layer F.Cu) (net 17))
 (segment (start 74.168 138.176) (end 76.2 138.176) (width 0.25) (layer F.Cu) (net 6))
 (segment (start 74.168 159.766) (end 74.168 138.176) (width 0.25) (layer F.Cu) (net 6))
 (segment (start 94.234 156.972) (end 94.234 165.989) (width 0.25) (layer F.Cu) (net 6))
 (segment (start 95.377 156.972) (end 94.234 156.972) (width 0.25) (layer F.Cu) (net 6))
 (segment (start 94.234 165.989) (end 88.9 165.989) (width 0.25) (layer F.Cu) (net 6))
 (segment (start 88.9 165.989) (end 88.9 164.846) (width 0.25) (layer F.Cu) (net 6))
 (segment (start 88.9 164.846) (end 78.74 164.846) (width 0.25) (layer F.Cu) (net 6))
 (segment (start 78.74 159.766) (end 74.168 159.766) (width 0.25) (layer F.Cu) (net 6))
 (segment (start 78.74 164.846) (end 78.74 159.766) (width 0.25) (layer F.Cu) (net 6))
 (segment (start 112.736 163.451) (end 112.736 163.576) (width 0.25) (layer B.Cu) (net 6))
 (segment (start 111.379 161.163) (end 112.736 163.451) (width 0.25) (layer B.Cu) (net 6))
 (segment (start 95.377 157.099) (end 96.774 161.163) (width 0.25) (layer B.Cu) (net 6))
 (segment (start 96.774 161.163) (end 111.379 161.163) (width 0.25) (layer B.Cu) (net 6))
 (segment (start 132.66 143.654213) (end 132.66 148.74) (width 0.25) (layer F.Cu) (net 4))
 (segment (start 132.66 142.24) (end 132.66 143.654213) (width 0.25) (layer F.Cu) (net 4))
 (segment (start 130.81 150.59) (end 130.81 154.94) (width 0.25) (layer F.Cu) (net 4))
 (segment (start 132.66 148.74) (end 130.81 150.59) (width 0.25) (layer F.Cu) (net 4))
 (segment (start 130.81 155.929949) (end 130.81 158.75) (width 0.25) (layer F.Cu) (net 4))
 (segment (start 130.81 154.94) (end 130.81 155.929949) (width 0.25) (layer F.Cu) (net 4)))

